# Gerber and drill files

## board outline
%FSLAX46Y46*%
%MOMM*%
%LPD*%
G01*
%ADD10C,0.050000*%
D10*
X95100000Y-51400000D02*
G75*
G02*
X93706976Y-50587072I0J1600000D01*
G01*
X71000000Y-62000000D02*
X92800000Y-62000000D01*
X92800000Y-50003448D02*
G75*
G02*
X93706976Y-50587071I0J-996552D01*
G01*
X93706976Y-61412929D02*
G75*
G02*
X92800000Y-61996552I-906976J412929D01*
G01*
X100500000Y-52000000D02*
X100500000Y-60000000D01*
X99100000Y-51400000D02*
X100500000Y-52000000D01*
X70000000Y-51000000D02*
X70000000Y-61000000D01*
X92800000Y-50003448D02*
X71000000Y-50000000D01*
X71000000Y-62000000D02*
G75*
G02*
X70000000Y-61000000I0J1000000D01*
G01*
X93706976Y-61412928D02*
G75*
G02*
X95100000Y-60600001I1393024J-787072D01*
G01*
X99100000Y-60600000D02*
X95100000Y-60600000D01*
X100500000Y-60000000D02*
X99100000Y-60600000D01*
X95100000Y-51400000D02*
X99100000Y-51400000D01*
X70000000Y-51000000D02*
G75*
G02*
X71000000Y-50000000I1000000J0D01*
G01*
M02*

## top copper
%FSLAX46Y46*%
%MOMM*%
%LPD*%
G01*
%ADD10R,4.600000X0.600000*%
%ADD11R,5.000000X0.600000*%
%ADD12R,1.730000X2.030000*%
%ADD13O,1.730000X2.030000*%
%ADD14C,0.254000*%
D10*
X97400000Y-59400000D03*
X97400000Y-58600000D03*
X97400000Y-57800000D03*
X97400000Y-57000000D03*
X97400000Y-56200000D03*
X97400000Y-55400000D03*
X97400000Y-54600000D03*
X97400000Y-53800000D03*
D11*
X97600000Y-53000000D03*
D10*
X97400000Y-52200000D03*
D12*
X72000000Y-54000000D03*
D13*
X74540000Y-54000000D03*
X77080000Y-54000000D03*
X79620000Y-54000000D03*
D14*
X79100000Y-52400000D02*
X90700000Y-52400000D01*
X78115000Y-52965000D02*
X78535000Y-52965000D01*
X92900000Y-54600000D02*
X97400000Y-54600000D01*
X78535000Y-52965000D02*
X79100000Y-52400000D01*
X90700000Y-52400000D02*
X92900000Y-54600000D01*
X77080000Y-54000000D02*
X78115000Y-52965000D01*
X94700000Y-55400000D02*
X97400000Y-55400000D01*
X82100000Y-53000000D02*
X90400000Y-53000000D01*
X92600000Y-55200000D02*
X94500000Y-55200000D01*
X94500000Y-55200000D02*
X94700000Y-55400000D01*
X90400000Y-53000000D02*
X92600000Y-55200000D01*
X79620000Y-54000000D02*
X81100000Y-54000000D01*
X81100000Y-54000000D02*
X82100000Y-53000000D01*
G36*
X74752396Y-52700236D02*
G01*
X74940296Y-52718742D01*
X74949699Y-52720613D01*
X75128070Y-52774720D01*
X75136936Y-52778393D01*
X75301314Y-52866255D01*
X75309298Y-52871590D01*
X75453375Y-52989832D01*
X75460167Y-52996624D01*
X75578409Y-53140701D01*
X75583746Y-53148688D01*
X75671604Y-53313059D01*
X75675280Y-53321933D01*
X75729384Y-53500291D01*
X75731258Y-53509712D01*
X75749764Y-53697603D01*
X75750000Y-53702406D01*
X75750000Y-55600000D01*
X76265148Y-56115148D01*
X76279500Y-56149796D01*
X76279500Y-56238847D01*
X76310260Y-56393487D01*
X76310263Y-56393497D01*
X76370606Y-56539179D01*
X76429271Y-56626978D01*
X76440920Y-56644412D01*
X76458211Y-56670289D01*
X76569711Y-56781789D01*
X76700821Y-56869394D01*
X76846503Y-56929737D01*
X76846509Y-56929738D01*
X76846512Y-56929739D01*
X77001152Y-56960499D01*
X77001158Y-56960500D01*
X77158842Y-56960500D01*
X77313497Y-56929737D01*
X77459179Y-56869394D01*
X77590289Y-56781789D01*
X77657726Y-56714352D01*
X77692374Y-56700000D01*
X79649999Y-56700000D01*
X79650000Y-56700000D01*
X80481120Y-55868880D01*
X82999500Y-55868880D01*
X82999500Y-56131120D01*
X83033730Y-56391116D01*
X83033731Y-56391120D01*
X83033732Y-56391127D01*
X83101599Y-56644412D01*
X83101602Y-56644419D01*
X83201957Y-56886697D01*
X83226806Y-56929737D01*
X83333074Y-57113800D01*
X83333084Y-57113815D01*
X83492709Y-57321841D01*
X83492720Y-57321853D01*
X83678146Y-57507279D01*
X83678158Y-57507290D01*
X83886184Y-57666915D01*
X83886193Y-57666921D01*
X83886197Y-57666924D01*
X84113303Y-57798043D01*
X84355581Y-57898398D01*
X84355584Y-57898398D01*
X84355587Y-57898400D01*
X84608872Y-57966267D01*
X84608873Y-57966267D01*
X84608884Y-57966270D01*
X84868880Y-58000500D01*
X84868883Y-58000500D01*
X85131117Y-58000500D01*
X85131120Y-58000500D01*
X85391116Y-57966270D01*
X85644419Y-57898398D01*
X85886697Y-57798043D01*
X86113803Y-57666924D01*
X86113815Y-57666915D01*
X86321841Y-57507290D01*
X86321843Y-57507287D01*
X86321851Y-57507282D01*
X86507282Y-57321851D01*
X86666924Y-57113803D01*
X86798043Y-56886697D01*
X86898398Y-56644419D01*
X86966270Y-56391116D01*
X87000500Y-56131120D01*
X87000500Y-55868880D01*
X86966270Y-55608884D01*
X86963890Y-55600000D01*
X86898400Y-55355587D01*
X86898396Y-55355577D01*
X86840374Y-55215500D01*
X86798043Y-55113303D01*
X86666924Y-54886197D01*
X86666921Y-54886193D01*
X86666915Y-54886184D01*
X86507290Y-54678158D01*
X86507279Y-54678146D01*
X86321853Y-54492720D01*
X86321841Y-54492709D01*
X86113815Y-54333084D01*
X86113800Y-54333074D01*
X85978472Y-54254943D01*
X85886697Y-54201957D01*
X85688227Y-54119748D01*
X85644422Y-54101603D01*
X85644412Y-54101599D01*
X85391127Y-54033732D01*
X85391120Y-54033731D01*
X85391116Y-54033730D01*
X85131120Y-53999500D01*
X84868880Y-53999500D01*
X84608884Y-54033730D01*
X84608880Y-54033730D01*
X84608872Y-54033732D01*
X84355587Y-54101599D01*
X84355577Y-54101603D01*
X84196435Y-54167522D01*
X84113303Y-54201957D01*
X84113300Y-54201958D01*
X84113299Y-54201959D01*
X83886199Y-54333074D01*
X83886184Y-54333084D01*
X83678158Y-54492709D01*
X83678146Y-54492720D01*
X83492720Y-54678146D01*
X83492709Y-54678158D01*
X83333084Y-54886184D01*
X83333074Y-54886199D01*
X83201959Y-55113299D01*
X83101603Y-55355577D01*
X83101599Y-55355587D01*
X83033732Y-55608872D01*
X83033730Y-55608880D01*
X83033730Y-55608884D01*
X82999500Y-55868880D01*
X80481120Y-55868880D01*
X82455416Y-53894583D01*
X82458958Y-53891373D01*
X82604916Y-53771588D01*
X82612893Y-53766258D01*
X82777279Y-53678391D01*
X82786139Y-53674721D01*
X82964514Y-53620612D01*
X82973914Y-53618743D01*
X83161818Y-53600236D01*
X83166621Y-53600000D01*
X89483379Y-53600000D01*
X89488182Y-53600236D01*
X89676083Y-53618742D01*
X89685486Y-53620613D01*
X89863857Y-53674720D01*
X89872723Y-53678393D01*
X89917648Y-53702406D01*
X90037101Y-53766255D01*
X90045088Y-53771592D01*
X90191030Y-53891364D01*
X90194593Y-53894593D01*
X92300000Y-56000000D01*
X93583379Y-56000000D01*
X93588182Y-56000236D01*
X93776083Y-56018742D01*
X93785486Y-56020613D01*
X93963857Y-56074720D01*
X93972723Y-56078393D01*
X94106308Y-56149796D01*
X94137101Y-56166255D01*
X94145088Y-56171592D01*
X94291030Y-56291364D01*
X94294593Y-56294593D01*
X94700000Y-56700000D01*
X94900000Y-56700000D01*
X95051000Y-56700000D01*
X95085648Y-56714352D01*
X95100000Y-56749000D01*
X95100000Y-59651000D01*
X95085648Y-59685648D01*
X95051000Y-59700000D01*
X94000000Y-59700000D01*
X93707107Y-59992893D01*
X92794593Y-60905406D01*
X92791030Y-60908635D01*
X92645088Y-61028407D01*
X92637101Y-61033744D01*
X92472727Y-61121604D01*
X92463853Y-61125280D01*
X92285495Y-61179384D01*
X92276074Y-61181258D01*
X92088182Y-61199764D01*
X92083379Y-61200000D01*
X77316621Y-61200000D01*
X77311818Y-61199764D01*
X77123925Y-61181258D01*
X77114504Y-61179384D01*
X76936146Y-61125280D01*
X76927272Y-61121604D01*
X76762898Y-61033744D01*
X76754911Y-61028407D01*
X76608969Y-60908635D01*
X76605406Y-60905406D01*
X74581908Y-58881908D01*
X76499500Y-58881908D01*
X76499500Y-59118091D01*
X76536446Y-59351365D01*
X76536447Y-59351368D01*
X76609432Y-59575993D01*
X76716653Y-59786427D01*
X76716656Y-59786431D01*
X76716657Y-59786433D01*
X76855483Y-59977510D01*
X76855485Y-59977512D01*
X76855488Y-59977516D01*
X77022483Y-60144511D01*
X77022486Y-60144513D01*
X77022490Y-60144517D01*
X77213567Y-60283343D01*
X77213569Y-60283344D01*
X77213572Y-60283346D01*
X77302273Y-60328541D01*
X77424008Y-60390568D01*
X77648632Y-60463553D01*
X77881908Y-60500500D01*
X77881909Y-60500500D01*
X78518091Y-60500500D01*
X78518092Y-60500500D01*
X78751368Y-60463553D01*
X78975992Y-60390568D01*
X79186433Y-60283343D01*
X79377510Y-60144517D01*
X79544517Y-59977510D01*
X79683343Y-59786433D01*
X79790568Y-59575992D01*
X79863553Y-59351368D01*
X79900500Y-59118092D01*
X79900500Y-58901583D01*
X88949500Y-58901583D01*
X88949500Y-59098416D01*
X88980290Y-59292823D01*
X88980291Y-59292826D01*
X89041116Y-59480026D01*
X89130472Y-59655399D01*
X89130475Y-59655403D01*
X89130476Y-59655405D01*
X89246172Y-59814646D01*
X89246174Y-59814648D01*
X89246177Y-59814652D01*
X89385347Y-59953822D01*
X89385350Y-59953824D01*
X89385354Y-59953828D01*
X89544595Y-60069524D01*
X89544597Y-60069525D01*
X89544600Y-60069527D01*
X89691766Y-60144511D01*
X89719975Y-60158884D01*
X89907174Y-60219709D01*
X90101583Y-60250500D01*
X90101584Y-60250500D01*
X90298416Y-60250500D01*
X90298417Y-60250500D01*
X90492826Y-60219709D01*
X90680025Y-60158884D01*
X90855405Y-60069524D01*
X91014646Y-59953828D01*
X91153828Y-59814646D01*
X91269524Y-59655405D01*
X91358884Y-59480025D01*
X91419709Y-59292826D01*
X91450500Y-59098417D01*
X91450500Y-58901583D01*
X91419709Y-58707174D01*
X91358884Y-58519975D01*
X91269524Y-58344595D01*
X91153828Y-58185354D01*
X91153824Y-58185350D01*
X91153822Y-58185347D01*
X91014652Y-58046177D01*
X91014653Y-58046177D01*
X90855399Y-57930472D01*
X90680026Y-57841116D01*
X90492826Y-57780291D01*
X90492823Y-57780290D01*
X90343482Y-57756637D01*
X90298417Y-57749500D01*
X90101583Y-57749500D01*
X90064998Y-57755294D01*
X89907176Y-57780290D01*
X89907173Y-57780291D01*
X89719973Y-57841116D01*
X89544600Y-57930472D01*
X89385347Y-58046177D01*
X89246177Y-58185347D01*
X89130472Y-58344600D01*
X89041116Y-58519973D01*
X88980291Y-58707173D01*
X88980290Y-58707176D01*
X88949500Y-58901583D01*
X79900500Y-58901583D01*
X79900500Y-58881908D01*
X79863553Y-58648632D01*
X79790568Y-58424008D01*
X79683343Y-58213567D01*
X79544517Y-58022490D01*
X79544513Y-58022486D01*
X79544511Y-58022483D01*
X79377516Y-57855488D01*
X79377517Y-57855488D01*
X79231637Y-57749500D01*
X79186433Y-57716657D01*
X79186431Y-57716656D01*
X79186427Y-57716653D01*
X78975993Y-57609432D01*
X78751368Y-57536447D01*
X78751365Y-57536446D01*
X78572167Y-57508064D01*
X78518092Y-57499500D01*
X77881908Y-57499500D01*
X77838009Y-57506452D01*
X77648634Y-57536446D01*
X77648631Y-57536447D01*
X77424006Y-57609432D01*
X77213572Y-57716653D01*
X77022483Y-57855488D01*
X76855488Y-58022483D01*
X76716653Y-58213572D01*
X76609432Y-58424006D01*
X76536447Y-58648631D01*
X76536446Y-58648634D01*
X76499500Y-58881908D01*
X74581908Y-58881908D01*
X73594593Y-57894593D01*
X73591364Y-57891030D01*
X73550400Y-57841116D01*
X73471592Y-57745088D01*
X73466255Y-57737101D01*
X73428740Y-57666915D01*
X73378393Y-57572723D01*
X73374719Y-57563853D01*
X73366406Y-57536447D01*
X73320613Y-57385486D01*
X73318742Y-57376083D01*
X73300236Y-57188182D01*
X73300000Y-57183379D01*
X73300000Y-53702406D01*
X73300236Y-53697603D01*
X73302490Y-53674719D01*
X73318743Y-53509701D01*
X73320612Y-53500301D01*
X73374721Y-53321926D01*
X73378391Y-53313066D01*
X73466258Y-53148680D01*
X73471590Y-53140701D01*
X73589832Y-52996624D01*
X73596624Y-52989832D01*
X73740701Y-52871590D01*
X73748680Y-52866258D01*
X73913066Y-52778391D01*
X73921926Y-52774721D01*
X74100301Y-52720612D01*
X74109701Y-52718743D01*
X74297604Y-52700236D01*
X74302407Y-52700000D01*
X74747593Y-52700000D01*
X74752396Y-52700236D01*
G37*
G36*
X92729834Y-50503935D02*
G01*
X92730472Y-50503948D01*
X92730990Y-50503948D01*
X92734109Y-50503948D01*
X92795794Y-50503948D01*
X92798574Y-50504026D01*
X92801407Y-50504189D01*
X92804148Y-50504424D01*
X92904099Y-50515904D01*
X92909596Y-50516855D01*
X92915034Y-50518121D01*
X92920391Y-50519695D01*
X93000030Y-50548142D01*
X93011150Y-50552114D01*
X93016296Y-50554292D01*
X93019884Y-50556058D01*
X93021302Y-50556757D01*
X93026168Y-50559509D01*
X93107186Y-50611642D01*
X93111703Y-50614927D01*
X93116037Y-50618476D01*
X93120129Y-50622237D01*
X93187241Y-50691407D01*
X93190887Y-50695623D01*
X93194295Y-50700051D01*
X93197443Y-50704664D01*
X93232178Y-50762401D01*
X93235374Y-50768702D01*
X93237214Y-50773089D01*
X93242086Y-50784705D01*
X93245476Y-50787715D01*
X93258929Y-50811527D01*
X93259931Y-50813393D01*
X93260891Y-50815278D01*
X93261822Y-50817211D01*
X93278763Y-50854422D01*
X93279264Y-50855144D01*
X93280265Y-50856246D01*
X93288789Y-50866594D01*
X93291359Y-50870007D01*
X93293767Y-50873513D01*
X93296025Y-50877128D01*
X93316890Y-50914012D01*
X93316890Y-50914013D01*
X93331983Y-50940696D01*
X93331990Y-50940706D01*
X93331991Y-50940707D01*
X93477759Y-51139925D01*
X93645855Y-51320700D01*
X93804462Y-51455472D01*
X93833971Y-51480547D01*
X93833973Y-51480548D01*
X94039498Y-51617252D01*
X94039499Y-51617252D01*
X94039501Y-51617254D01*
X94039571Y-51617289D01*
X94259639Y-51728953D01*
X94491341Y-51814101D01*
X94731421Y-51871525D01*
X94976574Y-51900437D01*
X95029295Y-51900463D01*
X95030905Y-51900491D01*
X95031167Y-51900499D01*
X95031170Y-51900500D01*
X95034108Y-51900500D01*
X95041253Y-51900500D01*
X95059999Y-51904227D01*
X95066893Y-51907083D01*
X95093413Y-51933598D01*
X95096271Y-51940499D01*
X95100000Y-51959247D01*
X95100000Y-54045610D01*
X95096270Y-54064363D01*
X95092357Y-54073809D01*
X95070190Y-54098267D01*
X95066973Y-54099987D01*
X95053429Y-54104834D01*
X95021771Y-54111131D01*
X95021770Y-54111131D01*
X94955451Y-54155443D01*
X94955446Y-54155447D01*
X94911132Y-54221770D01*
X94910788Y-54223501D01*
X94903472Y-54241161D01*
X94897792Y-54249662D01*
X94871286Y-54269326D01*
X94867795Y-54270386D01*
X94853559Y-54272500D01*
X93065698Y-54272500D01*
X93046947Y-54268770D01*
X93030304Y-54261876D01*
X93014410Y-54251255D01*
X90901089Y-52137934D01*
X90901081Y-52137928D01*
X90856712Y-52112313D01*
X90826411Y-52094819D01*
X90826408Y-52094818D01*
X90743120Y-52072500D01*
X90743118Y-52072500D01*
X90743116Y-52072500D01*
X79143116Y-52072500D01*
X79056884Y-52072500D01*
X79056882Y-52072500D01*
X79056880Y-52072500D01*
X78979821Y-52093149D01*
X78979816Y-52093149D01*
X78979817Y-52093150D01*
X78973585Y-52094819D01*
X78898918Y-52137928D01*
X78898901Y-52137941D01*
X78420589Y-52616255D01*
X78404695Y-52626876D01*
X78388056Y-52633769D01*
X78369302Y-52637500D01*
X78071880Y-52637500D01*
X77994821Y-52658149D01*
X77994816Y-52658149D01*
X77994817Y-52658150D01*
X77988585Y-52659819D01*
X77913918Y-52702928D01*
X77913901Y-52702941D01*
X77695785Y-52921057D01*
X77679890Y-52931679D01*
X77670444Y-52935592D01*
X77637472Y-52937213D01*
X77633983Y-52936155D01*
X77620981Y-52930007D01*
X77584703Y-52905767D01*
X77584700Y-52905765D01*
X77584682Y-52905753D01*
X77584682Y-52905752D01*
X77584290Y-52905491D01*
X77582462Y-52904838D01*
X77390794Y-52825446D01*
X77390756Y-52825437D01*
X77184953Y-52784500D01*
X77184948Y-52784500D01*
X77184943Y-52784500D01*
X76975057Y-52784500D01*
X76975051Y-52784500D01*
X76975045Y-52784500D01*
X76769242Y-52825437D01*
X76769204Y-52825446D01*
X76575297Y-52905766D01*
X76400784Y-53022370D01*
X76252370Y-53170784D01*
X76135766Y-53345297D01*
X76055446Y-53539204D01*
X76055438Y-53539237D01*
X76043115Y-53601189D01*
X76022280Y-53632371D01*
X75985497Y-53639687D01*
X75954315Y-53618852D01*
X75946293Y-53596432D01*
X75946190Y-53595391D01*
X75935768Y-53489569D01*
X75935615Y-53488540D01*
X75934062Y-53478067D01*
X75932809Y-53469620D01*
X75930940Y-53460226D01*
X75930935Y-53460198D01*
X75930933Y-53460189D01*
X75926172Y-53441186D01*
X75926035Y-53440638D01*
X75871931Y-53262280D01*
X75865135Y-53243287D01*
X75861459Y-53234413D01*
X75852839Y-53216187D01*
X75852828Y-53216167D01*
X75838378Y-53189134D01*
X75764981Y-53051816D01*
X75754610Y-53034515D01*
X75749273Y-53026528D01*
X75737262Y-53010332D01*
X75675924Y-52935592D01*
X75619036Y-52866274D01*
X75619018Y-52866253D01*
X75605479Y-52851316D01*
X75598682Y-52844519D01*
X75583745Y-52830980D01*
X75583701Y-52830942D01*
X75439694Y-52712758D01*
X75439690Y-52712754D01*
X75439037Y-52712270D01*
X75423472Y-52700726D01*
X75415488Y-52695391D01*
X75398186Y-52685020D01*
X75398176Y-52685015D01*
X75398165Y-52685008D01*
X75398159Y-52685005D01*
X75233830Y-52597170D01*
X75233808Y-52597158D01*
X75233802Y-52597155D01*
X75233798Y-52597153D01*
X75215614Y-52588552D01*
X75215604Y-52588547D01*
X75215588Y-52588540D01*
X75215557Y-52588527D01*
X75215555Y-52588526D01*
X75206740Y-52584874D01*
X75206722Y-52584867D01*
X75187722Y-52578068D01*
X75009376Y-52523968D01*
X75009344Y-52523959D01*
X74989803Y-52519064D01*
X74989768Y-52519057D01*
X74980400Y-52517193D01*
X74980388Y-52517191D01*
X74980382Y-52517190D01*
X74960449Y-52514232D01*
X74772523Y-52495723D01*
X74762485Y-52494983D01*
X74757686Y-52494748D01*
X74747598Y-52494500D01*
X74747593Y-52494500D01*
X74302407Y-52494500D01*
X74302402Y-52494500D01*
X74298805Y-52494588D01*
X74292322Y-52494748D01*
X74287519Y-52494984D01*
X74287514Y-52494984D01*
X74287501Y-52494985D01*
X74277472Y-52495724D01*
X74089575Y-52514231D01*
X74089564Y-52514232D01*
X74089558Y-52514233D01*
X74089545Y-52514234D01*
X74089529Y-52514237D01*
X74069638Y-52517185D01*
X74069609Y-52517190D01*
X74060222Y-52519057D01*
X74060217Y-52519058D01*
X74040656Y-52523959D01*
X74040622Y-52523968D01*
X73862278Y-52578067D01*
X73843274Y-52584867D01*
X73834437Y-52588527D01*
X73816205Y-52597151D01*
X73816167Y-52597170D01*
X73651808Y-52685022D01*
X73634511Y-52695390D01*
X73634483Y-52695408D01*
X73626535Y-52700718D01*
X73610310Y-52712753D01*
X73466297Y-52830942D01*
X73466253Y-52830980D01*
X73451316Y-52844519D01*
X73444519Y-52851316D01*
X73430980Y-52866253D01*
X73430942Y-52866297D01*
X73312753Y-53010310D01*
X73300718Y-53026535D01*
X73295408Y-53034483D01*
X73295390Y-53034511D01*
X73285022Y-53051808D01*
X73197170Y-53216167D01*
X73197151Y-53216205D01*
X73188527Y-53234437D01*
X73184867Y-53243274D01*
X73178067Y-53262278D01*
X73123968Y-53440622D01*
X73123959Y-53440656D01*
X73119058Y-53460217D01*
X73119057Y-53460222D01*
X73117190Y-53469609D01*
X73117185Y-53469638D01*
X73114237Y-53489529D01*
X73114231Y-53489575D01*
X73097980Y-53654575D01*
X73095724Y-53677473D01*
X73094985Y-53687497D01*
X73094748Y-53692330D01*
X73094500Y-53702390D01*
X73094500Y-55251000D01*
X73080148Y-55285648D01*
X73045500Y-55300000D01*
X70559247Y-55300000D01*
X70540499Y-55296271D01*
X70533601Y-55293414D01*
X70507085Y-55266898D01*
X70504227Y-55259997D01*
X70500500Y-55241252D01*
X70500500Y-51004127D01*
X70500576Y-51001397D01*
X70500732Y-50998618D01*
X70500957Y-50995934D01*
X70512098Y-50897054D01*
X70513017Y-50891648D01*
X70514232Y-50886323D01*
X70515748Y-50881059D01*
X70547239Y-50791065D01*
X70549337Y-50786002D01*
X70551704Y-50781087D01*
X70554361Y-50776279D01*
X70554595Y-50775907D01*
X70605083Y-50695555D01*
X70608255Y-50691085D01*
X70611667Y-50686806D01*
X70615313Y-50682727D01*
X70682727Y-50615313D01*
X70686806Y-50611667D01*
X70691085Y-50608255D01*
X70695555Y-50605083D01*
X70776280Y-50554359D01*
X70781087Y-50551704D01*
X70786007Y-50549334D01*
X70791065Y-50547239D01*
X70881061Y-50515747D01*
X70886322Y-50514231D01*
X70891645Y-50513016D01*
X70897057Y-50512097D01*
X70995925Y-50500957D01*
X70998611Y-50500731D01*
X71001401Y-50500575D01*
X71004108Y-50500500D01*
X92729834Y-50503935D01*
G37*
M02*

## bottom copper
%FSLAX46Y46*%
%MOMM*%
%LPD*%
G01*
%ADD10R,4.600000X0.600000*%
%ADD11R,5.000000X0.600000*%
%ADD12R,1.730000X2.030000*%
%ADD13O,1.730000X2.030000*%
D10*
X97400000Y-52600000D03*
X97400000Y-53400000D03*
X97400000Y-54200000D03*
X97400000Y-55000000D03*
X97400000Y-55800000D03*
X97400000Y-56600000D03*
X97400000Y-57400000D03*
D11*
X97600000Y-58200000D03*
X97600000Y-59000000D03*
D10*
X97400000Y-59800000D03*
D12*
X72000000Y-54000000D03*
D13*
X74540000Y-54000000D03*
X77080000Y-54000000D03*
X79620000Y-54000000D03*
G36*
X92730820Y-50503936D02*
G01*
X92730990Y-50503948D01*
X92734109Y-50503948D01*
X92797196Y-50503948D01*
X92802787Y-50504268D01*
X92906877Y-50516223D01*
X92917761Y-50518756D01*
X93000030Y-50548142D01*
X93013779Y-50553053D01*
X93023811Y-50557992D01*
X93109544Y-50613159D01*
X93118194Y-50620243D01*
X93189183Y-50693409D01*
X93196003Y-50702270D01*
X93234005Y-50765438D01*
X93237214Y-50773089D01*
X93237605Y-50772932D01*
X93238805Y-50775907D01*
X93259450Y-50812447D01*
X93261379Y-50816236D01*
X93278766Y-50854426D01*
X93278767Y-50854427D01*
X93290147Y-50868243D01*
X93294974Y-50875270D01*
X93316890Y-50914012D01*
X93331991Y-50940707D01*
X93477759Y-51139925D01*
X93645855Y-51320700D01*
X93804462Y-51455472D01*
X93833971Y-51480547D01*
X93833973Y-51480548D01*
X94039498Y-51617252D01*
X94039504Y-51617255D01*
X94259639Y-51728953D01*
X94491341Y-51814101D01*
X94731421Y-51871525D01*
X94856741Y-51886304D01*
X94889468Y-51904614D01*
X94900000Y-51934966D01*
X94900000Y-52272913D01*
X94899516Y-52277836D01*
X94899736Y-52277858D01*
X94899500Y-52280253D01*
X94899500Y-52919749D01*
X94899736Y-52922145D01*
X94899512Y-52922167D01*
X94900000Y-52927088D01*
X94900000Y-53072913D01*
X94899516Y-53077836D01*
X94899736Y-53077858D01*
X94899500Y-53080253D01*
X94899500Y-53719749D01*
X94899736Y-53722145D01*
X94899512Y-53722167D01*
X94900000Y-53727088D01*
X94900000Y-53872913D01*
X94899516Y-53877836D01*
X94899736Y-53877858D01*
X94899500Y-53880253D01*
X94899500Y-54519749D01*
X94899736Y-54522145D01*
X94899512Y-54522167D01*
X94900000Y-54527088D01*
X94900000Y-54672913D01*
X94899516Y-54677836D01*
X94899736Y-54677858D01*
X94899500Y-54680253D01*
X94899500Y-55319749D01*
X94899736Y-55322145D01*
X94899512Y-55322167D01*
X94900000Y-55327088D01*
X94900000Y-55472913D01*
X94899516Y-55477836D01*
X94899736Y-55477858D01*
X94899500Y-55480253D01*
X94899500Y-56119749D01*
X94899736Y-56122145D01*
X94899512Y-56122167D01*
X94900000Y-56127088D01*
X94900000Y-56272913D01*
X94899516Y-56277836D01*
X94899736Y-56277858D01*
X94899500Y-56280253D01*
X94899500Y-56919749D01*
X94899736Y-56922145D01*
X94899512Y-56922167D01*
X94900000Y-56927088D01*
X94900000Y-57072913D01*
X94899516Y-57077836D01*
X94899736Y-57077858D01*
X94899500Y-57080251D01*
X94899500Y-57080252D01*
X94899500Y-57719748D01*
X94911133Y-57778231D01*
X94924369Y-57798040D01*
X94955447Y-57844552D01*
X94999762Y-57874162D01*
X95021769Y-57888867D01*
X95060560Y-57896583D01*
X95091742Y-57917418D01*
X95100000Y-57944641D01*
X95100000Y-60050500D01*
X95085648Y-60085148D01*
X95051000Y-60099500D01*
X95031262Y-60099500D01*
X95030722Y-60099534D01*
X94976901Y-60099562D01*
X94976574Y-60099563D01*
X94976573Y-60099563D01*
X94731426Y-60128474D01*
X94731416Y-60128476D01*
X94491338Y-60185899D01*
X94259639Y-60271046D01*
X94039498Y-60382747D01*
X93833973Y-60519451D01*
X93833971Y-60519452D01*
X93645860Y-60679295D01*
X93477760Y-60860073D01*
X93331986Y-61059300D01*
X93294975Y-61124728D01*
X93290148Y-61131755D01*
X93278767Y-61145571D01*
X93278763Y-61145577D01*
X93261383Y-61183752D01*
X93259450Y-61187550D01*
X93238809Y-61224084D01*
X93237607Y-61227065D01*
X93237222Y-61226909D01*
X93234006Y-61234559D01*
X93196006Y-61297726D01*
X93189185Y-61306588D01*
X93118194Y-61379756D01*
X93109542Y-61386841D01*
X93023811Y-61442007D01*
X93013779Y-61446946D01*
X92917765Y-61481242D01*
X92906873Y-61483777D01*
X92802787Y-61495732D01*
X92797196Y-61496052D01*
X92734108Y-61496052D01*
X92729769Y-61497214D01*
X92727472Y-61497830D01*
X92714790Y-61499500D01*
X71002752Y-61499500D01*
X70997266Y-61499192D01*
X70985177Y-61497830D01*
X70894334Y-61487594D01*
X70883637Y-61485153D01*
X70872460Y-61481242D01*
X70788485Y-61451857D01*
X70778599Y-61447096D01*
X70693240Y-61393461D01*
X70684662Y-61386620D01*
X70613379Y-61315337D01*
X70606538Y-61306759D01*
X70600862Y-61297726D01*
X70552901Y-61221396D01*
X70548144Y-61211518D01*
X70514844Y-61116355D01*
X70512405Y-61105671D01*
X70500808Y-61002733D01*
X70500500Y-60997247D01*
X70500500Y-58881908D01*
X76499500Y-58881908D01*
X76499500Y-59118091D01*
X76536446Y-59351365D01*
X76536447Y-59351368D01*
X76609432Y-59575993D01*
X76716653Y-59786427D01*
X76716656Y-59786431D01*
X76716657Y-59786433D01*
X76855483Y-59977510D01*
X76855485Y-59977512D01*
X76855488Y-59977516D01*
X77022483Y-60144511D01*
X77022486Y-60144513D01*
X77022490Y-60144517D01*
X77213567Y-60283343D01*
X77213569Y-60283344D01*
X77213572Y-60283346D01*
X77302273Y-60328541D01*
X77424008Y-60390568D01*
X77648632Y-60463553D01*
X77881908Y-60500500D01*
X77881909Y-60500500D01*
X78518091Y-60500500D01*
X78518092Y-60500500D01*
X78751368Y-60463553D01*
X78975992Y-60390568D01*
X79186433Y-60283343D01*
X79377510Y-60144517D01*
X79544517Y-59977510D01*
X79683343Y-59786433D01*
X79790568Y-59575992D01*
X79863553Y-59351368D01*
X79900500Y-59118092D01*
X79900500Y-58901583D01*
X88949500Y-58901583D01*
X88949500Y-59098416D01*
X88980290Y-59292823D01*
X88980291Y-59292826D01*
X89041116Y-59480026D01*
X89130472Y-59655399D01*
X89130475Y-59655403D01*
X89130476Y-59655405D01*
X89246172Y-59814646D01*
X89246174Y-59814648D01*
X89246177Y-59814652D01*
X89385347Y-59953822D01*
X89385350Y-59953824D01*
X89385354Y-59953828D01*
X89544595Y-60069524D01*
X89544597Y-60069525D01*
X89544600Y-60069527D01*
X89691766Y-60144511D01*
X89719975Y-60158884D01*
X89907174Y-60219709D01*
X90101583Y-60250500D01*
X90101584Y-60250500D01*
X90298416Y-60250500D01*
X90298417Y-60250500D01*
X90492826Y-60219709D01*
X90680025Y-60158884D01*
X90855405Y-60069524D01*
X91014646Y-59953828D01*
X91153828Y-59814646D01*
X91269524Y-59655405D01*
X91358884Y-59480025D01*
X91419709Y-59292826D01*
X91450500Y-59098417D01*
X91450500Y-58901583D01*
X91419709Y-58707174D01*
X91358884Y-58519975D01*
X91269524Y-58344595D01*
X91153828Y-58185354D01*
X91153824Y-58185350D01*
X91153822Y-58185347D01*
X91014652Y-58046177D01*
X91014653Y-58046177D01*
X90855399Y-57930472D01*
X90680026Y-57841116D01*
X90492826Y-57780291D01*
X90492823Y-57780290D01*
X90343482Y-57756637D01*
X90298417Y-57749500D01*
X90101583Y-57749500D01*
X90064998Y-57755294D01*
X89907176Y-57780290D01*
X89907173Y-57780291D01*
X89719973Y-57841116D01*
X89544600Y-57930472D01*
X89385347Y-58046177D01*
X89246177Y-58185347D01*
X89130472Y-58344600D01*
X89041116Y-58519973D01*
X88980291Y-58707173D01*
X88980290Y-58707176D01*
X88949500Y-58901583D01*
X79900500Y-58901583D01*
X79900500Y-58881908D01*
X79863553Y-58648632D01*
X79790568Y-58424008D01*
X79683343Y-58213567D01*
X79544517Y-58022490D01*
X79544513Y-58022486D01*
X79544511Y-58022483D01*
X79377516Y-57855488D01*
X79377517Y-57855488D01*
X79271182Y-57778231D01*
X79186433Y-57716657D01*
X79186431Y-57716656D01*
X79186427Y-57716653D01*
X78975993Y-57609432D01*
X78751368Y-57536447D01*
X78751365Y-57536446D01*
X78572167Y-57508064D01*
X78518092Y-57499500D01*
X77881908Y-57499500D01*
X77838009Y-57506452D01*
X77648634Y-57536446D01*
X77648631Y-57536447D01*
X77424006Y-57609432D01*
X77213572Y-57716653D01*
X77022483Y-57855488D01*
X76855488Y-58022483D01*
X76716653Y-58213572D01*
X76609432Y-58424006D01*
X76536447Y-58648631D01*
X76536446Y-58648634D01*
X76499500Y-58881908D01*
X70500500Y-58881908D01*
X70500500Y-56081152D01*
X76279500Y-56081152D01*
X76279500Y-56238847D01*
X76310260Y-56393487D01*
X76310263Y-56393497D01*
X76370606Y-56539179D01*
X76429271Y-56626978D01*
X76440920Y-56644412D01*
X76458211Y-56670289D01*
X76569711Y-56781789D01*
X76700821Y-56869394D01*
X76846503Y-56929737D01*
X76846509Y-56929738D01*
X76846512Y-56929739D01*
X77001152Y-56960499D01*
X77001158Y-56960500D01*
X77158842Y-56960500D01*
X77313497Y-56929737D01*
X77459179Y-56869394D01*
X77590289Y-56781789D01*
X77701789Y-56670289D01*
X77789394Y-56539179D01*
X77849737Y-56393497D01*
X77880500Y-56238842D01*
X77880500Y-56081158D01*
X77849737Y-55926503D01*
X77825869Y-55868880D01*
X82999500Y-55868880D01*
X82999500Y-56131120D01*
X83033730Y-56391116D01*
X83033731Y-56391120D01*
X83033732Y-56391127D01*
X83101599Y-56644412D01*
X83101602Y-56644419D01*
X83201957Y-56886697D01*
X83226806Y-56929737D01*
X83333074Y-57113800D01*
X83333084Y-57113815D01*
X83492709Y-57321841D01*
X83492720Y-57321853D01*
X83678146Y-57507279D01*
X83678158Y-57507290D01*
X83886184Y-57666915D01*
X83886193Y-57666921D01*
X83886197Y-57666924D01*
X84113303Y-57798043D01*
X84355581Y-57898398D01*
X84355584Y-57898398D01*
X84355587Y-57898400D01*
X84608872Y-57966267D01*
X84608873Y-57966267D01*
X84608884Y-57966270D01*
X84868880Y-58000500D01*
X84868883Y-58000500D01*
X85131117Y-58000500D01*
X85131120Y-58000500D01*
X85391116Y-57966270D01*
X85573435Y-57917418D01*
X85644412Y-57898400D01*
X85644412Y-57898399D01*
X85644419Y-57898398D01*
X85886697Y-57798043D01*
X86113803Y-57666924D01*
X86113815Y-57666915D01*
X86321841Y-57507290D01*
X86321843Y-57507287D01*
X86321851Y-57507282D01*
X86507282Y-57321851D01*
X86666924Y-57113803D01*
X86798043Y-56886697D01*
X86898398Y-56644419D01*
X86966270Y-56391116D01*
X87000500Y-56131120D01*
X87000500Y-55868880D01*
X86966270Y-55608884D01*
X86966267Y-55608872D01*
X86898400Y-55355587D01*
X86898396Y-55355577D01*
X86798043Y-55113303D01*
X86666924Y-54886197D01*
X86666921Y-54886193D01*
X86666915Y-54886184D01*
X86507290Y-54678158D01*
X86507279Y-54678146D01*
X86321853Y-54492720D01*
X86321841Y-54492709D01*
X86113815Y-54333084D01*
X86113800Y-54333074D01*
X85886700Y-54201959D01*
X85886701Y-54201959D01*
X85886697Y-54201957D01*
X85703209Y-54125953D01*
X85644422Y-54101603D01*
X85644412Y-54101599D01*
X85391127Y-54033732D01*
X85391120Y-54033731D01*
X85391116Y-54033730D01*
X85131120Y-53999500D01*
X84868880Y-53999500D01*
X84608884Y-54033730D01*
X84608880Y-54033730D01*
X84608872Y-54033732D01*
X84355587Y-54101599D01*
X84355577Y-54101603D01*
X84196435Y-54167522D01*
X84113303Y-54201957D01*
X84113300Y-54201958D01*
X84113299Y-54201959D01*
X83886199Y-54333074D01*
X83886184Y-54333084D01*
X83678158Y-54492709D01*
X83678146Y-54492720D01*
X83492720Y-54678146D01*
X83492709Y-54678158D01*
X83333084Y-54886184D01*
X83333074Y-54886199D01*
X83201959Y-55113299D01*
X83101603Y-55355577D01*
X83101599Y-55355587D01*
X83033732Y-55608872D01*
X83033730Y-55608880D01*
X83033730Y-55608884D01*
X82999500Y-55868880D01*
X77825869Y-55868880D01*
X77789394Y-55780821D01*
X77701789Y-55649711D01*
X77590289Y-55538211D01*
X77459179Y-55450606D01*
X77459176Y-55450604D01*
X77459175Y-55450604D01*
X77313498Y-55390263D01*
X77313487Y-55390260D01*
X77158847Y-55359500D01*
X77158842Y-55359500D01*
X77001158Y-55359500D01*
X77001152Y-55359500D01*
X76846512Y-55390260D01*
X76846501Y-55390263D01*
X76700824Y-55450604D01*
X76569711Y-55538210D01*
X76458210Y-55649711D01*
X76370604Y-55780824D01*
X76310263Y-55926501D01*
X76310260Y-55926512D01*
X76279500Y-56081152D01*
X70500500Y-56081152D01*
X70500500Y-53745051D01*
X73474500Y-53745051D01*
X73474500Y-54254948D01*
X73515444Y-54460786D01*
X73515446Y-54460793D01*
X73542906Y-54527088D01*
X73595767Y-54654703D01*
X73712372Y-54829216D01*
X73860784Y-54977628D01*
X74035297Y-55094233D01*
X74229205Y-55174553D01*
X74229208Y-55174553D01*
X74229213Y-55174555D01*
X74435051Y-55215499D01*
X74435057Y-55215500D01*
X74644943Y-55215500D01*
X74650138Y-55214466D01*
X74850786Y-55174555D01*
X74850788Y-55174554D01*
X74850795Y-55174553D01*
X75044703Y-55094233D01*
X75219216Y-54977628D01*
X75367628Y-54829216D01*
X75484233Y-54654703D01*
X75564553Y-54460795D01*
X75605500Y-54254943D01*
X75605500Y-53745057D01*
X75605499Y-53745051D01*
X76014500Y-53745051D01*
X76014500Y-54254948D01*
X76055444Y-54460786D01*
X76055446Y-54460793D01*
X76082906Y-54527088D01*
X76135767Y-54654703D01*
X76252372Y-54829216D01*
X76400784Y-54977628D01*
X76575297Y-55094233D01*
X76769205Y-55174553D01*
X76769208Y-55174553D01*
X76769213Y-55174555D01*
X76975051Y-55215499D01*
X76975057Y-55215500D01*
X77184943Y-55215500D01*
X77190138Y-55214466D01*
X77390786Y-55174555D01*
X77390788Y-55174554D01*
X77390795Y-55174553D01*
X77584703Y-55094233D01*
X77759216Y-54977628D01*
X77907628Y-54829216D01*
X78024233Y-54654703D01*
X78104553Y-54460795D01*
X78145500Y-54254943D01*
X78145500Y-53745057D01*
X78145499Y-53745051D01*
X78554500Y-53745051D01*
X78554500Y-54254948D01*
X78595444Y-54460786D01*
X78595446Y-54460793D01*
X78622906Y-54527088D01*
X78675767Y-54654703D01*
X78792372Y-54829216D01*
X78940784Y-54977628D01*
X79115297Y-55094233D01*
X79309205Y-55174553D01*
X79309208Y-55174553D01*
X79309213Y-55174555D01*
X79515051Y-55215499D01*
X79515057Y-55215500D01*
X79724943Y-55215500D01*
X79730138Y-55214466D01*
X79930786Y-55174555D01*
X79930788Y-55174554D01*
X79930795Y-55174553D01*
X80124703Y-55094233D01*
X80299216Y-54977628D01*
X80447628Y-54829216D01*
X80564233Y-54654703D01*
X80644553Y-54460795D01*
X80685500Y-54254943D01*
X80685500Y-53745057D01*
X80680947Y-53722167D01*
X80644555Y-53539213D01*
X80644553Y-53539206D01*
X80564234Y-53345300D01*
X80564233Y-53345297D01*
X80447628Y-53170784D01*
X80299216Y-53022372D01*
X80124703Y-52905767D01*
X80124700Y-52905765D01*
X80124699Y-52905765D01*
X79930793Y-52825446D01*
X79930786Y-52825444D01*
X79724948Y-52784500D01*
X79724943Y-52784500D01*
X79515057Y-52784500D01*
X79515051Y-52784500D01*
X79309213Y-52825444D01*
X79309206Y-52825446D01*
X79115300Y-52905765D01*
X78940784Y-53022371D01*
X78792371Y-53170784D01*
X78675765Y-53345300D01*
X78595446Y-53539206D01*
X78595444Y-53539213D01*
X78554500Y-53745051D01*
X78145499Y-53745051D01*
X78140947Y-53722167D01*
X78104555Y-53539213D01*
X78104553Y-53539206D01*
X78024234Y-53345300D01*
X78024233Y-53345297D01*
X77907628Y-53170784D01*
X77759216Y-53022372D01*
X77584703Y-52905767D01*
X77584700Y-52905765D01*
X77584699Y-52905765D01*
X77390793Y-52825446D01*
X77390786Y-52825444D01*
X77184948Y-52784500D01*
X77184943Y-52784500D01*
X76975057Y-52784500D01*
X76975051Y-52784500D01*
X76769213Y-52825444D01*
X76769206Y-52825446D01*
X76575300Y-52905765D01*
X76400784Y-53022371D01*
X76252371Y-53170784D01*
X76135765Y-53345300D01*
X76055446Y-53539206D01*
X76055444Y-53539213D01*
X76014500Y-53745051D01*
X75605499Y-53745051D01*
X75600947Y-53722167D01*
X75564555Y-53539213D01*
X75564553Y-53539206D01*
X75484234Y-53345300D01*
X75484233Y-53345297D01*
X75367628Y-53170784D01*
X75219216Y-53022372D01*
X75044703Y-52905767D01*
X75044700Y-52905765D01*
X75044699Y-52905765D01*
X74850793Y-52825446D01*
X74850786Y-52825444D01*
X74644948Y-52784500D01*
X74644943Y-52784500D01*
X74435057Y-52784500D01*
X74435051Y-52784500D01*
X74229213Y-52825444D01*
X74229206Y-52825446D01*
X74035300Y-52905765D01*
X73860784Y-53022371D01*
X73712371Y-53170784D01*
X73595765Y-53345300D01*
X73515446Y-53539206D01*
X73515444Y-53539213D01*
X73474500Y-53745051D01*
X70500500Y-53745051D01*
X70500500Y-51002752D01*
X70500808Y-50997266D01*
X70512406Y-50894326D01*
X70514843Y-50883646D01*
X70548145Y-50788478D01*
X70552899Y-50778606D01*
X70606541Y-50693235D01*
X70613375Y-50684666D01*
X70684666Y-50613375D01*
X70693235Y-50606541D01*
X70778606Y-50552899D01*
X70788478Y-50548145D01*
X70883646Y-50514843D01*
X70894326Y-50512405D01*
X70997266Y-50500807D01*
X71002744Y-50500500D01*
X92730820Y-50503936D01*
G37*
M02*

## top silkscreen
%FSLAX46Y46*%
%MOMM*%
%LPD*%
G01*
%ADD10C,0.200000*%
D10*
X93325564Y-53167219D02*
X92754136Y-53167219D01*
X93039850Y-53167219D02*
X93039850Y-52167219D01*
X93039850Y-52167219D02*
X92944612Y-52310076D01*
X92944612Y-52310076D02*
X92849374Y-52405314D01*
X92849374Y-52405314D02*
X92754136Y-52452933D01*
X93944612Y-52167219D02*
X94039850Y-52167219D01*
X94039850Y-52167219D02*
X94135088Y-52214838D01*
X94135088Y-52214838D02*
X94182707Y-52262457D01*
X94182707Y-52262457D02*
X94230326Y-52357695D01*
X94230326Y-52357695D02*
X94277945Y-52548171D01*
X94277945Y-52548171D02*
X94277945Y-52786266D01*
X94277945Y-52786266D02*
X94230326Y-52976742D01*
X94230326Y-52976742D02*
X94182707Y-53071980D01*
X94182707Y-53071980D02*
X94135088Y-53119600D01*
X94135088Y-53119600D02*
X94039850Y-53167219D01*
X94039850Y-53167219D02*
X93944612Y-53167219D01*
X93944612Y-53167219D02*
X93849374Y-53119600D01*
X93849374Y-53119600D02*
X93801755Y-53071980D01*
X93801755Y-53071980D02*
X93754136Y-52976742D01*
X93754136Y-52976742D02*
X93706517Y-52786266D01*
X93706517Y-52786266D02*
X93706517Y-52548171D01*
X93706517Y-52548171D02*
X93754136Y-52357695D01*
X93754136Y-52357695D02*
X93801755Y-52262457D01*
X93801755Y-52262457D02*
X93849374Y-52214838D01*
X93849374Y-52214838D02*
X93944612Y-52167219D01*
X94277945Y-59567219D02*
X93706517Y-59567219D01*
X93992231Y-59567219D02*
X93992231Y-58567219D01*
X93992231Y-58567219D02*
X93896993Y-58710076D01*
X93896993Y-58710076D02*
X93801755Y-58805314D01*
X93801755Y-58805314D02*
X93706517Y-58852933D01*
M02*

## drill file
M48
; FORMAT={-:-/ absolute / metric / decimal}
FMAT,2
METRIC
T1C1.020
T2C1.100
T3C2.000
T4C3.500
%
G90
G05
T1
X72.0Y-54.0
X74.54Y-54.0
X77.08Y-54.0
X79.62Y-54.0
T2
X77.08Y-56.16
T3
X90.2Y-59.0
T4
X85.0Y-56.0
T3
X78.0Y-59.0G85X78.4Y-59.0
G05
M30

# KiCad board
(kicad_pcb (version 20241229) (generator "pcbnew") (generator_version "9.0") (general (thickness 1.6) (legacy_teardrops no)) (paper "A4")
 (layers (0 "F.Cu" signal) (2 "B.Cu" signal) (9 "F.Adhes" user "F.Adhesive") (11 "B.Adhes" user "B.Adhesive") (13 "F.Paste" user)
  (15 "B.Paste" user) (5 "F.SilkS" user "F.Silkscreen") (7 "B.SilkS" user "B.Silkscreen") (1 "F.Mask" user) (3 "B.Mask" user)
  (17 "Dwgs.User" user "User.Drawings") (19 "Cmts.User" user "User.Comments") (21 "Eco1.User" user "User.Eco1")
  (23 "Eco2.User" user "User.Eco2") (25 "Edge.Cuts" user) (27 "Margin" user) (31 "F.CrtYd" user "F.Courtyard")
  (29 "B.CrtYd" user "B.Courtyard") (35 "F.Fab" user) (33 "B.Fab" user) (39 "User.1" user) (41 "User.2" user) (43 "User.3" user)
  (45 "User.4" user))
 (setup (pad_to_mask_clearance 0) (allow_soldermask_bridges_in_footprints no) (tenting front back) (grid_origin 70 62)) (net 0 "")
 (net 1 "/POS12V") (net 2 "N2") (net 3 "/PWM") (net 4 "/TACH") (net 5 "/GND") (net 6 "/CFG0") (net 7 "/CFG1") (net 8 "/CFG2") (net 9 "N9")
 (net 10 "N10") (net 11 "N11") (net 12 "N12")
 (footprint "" (layer "F.Cu") (at 80.2 64.4)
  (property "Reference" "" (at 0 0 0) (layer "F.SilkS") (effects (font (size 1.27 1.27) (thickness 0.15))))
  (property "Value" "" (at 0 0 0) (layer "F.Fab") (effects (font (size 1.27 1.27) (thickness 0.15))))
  (pad "" np_thru_hole circle (at 10 -5.4) (size 2 2) (drill 2) (layers "*.Cu" "*.Mask")))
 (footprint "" (layer "F.Cu") (at 81.7 44.8)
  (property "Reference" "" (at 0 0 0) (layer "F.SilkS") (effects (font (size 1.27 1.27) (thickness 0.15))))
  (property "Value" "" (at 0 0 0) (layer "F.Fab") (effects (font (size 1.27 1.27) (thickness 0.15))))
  (pad "" np_thru_hole oval (at -3.5 14.2) (size 2.4 2) (drill oval 2.4 2) (layers "*.Cu" "*.Mask")))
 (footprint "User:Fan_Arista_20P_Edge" (layer "F.Cu") (at 95.1 56)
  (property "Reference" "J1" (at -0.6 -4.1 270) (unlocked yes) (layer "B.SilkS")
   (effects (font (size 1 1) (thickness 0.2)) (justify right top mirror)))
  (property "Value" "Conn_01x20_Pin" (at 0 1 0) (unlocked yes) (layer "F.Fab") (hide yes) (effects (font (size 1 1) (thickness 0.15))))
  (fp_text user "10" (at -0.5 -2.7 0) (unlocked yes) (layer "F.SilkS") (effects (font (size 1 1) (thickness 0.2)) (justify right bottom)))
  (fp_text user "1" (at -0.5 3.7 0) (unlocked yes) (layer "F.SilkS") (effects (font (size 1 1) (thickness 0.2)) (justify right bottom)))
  (pad "1" connect rect (at 2.3 3.4) (size 4.6 0.6) (layers "F.Cu") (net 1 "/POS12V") (thermal_bridge_angle 45))
  (pad "2" connect rect (at 2.3 2.6) (size 4.6 0.6) (layers "F.Cu") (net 1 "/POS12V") (thermal_bridge_angle 45))
  (pad "3" connect rect (at 2.3 1.8) (size 4.6 0.6) (layers "F.Cu") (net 1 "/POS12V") (thermal_bridge_angle 45))
  (pad "4" connect rect (at 2.3 1) (size 4.6 0.6) (layers "F.Cu") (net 1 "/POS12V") (thermal_bridge_angle 45))
  (pad "5" connect rect (at 2.3 0.2) (size 4.6 0.6) (layers "F.Cu") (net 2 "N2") (thermal_bridge_angle 45))
  (pad "6" connect rect (at 2.3 -0.6) (size 4.6 0.6) (layers "F.Cu") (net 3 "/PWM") (thermal_bridge_angle 45))
  (pad "7" connect rect (at 2.3 -1.4) (size 4.6 0.6) (layers "F.Cu") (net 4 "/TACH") (thermal_bridge_angle 45))
  (pad "8" connect rect (at 2.3 -2.2) (size 4.6 0.6) (layers "F.Cu") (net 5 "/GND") (thermal_bridge_angle 45))
  (pad "9" connect rect (at 2.5 -3) (size 5 0.6) (layers "F.Cu") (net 5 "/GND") (thermal_bridge_angle 45))
  (pad "10" connect rect (at 2.3 -3.8) (size 4.6 0.6) (layers "F.Cu") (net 5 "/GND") (thermal_bridge_angle 45))
  (pad "11" connect rect (at 2.3 -3.4) (size 4.6 0.6) (layers "B.Cu") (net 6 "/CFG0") (thermal_bridge_angle 45))
  (pad "12" connect rect (at 2.3 -2.6) (size 4.6 0.6) (layers "B.Cu") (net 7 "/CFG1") (thermal_bridge_angle 45))
  (pad "13" connect rect (at 2.3 -1.8) (size 4.6 0.6) (layers "B.Cu") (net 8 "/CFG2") (thermal_bridge_angle 45))
  (pad "14" connect rect (at 2.3 -1) (size 4.6 0.6) (layers "B.Cu") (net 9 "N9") (thermal_bridge_angle 45))
  (pad "15" connect rect (at 2.3 -0.2) (size 4.6 0.6) (layers "B.Cu") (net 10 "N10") (thermal_bridge_angle 45))
  (pad "16" connect rect (at 2.3 0.6) (size 4.6 0.6) (layers "B.Cu") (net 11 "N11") (thermal_bridge_angle 45))
  (pad "17" connect rect (at 2.3 1.4) (size 4.6 0.6) (layers "B.Cu") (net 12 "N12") (thermal_bridge_angle 45))
  (pad "18" connect rect (at 2.5 2.2) (size 5 0.6) (layers "B.Cu") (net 5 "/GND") (thermal_bridge_angle 45))
  (pad "19" connect rect (at 2.5 3) (size 5 0.6) (layers "B.Cu") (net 5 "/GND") (thermal_bridge_angle 45))
  (pad "20" connect rect (at 2.3 3.8) (size 4.6 0.6) (layers "B.Cu") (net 5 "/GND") (thermal_bridge_angle 45))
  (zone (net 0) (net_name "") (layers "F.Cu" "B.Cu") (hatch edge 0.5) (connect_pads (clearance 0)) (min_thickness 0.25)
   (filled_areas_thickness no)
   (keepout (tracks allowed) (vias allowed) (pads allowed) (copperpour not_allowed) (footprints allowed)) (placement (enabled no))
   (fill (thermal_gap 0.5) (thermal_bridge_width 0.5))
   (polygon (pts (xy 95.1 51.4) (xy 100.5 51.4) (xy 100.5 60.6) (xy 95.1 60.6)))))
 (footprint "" (layer "F.Cu") (at 85 56)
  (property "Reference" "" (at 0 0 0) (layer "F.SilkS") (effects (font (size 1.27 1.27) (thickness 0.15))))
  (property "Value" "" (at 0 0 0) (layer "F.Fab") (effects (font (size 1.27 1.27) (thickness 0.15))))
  (pad "" np_thru_hole circle (at 0 0) (size 3.5 3.5) (drill 3.5) (layers "*.Cu" "*.Mask")))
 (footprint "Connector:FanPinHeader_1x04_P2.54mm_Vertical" (layer "B.Cu") (at 72 54)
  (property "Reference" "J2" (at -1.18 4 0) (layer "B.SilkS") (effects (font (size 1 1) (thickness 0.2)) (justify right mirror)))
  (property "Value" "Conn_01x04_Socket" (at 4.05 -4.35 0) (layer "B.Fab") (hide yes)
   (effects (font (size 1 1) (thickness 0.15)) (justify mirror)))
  (pad "" np_thru_hole circle (at 5.08 2.16 270) (size 1.1 1.1) (drill 1.1) (layers "*.Cu" "*.Mask"))
  (pad "1" thru_hole rect (at 0 0 270) (size 2.03 1.73) (drill 1.02) (layers "*.Cu" "*.Mask") (remove_unused_layers no) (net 5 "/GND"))
  (pad "2" thru_hole oval (at 2.54 0 270) (size 2.03 1.73) (drill 1.02) (layers "*.Cu" "*.Mask") (remove_unused_layers no) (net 1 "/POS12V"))
  (pad "3" thru_hole oval (at 5.08 0 270) (size 2.03 1.73) (drill 1.02) (layers "*.Cu" "*.Mask") (remove_unused_layers no) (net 4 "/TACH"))
  (pad "4" thru_hole oval (at 7.62 0 270) (size 2.03 1.73) (drill 1.02) (layers "*.Cu" "*.Mask") (remove_unused_layers no) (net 3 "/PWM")))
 (gr_arc (start 95.1 51.4) (mid 94.293562 51.181903) (end 93.706976 50.587072) (stroke (width 0.05) (type default)) (layer "Edge.Cuts"))
 (gr_line (start 71 62) (end 92.8 62) (stroke (width 0.05) (type default)) (layer "Edge.Cuts"))
 (gr_arc (start 92.8 50.003448) (mid 93.339264 50.16196) (end 93.706976 50.587071) (stroke (width 0.05) (type default)) (layer "Edge.Cuts"))
 (gr_arc (start 93.706976 61.412929) (mid 93.339264 61.83804) (end 92.8 61.996552) (stroke (width 0.05) (type default)) (layer "Edge.Cuts"))
 (gr_line (start 100.5 52) (end 100.5 60) (stroke (width 0.05) (type default)) (layer "Edge.Cuts"))
 (gr_line (start 99.1 51.4) (end 100.5 52) (stroke (width 0.05) (type default)) (layer "Edge.Cuts"))
 (gr_line (start 70 51) (end 70 61) (stroke (width 0.05) (type default)) (layer "Edge.Cuts"))
 (gr_line (start 92.8 50.003448) (end 71 50) (stroke (width 0.05) (type default)) (layer "Edge.Cuts"))
 (gr_arc (start 71 62) (mid 70.292893 61.707107) (end 70 61) (stroke (width 0.05) (type default)) (layer "Edge.Cuts"))
 (gr_arc (start 93.706976 61.412928) (mid 94.293562 60.818097) (end 95.1 60.6) (stroke (width 0.05) (type default)) (layer "Edge.Cuts"))
 (gr_line (start 99.1 60.6) (end 95.1 60.6) (stroke (width 0.05) (type default)) (layer "Edge.Cuts"))
 (gr_line (start 100.5 60) (end 99.1 60.6) (stroke (width 0.05) (type default)) (layer "Edge.Cuts"))
 (gr_line (start 95.1 51.4) (end 99.1 51.4) (stroke (width 0.05) (type default)) (layer "Edge.Cuts"))
 (gr_arc (start 70 51) (mid 70.292893 50.292893) (end 71 50) (stroke (width 0.05) (type default)) (layer "Edge.Cuts"))
 (segment (start 79.1 52.4) (end 90.7 52.4) (width 0.254) (layer "F.Cu") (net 4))
 (segment (start 78.115 52.965) (end 78.535 52.965) (width 0.254) (layer "F.Cu") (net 4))
 (segment (start 92.9 54.6) (end 97.4 54.6) (width 0.254) (layer "F.Cu") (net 4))
 (segment (start 78.535 52.965) (end 79.1 52.4) (width 0.254) (layer "F.Cu") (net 4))
 (segment (start 90.7 52.4) (end 92.9 54.6) (width 0.254) (layer "F.Cu") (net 4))
 (segment (start 77.08 54) (end 78.115 52.965) (width 0.254) (layer "F.Cu") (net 4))
 (segment (start 94.7 55.4) (end 97.4 55.4) (width 0.254) (layer "F.Cu") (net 3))
 (segment (start 82.1 53) (end 90.4 53) (width 0.254) (layer "F.Cu") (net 3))
 (segment (start 92.6 55.2) (end 94.5 55.2) (width 0.254) (layer "F.Cu") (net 3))
 (segment (start 94.5 55.2) (end 94.7 55.4) (width 0.254) (layer "F.Cu") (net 3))
 (segment (start 90.4 53) (end 92.6 55.2) (width 0.254) (layer "F.Cu") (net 3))
 (segment (start 79.62 54) (end 81.1 54) (width 0.254) (layer "F.Cu") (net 3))
 (segment (start 81.1 54) (end 82.1 53) (width 0.254) (layer "F.Cu") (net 3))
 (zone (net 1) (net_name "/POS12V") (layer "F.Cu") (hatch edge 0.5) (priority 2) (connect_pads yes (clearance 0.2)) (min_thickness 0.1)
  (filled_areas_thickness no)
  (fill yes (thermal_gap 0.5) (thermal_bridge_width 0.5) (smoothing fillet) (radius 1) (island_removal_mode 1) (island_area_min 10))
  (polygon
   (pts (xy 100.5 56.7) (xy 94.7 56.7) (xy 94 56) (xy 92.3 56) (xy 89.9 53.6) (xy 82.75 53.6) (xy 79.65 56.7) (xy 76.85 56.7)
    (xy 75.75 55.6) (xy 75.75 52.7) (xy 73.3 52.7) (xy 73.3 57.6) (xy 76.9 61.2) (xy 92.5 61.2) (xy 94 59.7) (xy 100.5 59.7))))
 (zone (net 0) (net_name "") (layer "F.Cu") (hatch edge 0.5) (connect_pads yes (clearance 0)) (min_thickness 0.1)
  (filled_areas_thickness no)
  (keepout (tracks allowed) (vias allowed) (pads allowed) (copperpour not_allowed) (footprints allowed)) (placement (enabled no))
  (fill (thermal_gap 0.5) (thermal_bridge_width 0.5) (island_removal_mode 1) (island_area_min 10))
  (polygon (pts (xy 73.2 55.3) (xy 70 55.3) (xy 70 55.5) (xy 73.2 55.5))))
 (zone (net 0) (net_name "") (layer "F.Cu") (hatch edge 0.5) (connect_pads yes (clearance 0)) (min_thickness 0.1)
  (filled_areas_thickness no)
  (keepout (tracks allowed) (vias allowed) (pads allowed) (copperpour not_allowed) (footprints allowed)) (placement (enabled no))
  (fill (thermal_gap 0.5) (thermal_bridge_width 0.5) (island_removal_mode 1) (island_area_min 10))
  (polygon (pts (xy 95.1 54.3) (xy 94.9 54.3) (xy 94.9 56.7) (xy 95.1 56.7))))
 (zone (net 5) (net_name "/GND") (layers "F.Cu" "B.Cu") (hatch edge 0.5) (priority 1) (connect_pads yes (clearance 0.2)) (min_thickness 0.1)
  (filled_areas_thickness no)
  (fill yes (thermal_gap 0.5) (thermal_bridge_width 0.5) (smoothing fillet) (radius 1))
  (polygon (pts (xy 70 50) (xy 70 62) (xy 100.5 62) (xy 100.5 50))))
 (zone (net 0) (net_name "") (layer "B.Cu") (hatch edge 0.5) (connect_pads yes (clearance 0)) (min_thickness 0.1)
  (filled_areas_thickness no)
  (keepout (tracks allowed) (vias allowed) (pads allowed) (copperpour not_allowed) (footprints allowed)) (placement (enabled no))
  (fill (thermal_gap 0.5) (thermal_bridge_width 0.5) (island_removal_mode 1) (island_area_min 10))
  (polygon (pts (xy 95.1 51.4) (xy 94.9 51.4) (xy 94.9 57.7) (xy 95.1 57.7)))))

